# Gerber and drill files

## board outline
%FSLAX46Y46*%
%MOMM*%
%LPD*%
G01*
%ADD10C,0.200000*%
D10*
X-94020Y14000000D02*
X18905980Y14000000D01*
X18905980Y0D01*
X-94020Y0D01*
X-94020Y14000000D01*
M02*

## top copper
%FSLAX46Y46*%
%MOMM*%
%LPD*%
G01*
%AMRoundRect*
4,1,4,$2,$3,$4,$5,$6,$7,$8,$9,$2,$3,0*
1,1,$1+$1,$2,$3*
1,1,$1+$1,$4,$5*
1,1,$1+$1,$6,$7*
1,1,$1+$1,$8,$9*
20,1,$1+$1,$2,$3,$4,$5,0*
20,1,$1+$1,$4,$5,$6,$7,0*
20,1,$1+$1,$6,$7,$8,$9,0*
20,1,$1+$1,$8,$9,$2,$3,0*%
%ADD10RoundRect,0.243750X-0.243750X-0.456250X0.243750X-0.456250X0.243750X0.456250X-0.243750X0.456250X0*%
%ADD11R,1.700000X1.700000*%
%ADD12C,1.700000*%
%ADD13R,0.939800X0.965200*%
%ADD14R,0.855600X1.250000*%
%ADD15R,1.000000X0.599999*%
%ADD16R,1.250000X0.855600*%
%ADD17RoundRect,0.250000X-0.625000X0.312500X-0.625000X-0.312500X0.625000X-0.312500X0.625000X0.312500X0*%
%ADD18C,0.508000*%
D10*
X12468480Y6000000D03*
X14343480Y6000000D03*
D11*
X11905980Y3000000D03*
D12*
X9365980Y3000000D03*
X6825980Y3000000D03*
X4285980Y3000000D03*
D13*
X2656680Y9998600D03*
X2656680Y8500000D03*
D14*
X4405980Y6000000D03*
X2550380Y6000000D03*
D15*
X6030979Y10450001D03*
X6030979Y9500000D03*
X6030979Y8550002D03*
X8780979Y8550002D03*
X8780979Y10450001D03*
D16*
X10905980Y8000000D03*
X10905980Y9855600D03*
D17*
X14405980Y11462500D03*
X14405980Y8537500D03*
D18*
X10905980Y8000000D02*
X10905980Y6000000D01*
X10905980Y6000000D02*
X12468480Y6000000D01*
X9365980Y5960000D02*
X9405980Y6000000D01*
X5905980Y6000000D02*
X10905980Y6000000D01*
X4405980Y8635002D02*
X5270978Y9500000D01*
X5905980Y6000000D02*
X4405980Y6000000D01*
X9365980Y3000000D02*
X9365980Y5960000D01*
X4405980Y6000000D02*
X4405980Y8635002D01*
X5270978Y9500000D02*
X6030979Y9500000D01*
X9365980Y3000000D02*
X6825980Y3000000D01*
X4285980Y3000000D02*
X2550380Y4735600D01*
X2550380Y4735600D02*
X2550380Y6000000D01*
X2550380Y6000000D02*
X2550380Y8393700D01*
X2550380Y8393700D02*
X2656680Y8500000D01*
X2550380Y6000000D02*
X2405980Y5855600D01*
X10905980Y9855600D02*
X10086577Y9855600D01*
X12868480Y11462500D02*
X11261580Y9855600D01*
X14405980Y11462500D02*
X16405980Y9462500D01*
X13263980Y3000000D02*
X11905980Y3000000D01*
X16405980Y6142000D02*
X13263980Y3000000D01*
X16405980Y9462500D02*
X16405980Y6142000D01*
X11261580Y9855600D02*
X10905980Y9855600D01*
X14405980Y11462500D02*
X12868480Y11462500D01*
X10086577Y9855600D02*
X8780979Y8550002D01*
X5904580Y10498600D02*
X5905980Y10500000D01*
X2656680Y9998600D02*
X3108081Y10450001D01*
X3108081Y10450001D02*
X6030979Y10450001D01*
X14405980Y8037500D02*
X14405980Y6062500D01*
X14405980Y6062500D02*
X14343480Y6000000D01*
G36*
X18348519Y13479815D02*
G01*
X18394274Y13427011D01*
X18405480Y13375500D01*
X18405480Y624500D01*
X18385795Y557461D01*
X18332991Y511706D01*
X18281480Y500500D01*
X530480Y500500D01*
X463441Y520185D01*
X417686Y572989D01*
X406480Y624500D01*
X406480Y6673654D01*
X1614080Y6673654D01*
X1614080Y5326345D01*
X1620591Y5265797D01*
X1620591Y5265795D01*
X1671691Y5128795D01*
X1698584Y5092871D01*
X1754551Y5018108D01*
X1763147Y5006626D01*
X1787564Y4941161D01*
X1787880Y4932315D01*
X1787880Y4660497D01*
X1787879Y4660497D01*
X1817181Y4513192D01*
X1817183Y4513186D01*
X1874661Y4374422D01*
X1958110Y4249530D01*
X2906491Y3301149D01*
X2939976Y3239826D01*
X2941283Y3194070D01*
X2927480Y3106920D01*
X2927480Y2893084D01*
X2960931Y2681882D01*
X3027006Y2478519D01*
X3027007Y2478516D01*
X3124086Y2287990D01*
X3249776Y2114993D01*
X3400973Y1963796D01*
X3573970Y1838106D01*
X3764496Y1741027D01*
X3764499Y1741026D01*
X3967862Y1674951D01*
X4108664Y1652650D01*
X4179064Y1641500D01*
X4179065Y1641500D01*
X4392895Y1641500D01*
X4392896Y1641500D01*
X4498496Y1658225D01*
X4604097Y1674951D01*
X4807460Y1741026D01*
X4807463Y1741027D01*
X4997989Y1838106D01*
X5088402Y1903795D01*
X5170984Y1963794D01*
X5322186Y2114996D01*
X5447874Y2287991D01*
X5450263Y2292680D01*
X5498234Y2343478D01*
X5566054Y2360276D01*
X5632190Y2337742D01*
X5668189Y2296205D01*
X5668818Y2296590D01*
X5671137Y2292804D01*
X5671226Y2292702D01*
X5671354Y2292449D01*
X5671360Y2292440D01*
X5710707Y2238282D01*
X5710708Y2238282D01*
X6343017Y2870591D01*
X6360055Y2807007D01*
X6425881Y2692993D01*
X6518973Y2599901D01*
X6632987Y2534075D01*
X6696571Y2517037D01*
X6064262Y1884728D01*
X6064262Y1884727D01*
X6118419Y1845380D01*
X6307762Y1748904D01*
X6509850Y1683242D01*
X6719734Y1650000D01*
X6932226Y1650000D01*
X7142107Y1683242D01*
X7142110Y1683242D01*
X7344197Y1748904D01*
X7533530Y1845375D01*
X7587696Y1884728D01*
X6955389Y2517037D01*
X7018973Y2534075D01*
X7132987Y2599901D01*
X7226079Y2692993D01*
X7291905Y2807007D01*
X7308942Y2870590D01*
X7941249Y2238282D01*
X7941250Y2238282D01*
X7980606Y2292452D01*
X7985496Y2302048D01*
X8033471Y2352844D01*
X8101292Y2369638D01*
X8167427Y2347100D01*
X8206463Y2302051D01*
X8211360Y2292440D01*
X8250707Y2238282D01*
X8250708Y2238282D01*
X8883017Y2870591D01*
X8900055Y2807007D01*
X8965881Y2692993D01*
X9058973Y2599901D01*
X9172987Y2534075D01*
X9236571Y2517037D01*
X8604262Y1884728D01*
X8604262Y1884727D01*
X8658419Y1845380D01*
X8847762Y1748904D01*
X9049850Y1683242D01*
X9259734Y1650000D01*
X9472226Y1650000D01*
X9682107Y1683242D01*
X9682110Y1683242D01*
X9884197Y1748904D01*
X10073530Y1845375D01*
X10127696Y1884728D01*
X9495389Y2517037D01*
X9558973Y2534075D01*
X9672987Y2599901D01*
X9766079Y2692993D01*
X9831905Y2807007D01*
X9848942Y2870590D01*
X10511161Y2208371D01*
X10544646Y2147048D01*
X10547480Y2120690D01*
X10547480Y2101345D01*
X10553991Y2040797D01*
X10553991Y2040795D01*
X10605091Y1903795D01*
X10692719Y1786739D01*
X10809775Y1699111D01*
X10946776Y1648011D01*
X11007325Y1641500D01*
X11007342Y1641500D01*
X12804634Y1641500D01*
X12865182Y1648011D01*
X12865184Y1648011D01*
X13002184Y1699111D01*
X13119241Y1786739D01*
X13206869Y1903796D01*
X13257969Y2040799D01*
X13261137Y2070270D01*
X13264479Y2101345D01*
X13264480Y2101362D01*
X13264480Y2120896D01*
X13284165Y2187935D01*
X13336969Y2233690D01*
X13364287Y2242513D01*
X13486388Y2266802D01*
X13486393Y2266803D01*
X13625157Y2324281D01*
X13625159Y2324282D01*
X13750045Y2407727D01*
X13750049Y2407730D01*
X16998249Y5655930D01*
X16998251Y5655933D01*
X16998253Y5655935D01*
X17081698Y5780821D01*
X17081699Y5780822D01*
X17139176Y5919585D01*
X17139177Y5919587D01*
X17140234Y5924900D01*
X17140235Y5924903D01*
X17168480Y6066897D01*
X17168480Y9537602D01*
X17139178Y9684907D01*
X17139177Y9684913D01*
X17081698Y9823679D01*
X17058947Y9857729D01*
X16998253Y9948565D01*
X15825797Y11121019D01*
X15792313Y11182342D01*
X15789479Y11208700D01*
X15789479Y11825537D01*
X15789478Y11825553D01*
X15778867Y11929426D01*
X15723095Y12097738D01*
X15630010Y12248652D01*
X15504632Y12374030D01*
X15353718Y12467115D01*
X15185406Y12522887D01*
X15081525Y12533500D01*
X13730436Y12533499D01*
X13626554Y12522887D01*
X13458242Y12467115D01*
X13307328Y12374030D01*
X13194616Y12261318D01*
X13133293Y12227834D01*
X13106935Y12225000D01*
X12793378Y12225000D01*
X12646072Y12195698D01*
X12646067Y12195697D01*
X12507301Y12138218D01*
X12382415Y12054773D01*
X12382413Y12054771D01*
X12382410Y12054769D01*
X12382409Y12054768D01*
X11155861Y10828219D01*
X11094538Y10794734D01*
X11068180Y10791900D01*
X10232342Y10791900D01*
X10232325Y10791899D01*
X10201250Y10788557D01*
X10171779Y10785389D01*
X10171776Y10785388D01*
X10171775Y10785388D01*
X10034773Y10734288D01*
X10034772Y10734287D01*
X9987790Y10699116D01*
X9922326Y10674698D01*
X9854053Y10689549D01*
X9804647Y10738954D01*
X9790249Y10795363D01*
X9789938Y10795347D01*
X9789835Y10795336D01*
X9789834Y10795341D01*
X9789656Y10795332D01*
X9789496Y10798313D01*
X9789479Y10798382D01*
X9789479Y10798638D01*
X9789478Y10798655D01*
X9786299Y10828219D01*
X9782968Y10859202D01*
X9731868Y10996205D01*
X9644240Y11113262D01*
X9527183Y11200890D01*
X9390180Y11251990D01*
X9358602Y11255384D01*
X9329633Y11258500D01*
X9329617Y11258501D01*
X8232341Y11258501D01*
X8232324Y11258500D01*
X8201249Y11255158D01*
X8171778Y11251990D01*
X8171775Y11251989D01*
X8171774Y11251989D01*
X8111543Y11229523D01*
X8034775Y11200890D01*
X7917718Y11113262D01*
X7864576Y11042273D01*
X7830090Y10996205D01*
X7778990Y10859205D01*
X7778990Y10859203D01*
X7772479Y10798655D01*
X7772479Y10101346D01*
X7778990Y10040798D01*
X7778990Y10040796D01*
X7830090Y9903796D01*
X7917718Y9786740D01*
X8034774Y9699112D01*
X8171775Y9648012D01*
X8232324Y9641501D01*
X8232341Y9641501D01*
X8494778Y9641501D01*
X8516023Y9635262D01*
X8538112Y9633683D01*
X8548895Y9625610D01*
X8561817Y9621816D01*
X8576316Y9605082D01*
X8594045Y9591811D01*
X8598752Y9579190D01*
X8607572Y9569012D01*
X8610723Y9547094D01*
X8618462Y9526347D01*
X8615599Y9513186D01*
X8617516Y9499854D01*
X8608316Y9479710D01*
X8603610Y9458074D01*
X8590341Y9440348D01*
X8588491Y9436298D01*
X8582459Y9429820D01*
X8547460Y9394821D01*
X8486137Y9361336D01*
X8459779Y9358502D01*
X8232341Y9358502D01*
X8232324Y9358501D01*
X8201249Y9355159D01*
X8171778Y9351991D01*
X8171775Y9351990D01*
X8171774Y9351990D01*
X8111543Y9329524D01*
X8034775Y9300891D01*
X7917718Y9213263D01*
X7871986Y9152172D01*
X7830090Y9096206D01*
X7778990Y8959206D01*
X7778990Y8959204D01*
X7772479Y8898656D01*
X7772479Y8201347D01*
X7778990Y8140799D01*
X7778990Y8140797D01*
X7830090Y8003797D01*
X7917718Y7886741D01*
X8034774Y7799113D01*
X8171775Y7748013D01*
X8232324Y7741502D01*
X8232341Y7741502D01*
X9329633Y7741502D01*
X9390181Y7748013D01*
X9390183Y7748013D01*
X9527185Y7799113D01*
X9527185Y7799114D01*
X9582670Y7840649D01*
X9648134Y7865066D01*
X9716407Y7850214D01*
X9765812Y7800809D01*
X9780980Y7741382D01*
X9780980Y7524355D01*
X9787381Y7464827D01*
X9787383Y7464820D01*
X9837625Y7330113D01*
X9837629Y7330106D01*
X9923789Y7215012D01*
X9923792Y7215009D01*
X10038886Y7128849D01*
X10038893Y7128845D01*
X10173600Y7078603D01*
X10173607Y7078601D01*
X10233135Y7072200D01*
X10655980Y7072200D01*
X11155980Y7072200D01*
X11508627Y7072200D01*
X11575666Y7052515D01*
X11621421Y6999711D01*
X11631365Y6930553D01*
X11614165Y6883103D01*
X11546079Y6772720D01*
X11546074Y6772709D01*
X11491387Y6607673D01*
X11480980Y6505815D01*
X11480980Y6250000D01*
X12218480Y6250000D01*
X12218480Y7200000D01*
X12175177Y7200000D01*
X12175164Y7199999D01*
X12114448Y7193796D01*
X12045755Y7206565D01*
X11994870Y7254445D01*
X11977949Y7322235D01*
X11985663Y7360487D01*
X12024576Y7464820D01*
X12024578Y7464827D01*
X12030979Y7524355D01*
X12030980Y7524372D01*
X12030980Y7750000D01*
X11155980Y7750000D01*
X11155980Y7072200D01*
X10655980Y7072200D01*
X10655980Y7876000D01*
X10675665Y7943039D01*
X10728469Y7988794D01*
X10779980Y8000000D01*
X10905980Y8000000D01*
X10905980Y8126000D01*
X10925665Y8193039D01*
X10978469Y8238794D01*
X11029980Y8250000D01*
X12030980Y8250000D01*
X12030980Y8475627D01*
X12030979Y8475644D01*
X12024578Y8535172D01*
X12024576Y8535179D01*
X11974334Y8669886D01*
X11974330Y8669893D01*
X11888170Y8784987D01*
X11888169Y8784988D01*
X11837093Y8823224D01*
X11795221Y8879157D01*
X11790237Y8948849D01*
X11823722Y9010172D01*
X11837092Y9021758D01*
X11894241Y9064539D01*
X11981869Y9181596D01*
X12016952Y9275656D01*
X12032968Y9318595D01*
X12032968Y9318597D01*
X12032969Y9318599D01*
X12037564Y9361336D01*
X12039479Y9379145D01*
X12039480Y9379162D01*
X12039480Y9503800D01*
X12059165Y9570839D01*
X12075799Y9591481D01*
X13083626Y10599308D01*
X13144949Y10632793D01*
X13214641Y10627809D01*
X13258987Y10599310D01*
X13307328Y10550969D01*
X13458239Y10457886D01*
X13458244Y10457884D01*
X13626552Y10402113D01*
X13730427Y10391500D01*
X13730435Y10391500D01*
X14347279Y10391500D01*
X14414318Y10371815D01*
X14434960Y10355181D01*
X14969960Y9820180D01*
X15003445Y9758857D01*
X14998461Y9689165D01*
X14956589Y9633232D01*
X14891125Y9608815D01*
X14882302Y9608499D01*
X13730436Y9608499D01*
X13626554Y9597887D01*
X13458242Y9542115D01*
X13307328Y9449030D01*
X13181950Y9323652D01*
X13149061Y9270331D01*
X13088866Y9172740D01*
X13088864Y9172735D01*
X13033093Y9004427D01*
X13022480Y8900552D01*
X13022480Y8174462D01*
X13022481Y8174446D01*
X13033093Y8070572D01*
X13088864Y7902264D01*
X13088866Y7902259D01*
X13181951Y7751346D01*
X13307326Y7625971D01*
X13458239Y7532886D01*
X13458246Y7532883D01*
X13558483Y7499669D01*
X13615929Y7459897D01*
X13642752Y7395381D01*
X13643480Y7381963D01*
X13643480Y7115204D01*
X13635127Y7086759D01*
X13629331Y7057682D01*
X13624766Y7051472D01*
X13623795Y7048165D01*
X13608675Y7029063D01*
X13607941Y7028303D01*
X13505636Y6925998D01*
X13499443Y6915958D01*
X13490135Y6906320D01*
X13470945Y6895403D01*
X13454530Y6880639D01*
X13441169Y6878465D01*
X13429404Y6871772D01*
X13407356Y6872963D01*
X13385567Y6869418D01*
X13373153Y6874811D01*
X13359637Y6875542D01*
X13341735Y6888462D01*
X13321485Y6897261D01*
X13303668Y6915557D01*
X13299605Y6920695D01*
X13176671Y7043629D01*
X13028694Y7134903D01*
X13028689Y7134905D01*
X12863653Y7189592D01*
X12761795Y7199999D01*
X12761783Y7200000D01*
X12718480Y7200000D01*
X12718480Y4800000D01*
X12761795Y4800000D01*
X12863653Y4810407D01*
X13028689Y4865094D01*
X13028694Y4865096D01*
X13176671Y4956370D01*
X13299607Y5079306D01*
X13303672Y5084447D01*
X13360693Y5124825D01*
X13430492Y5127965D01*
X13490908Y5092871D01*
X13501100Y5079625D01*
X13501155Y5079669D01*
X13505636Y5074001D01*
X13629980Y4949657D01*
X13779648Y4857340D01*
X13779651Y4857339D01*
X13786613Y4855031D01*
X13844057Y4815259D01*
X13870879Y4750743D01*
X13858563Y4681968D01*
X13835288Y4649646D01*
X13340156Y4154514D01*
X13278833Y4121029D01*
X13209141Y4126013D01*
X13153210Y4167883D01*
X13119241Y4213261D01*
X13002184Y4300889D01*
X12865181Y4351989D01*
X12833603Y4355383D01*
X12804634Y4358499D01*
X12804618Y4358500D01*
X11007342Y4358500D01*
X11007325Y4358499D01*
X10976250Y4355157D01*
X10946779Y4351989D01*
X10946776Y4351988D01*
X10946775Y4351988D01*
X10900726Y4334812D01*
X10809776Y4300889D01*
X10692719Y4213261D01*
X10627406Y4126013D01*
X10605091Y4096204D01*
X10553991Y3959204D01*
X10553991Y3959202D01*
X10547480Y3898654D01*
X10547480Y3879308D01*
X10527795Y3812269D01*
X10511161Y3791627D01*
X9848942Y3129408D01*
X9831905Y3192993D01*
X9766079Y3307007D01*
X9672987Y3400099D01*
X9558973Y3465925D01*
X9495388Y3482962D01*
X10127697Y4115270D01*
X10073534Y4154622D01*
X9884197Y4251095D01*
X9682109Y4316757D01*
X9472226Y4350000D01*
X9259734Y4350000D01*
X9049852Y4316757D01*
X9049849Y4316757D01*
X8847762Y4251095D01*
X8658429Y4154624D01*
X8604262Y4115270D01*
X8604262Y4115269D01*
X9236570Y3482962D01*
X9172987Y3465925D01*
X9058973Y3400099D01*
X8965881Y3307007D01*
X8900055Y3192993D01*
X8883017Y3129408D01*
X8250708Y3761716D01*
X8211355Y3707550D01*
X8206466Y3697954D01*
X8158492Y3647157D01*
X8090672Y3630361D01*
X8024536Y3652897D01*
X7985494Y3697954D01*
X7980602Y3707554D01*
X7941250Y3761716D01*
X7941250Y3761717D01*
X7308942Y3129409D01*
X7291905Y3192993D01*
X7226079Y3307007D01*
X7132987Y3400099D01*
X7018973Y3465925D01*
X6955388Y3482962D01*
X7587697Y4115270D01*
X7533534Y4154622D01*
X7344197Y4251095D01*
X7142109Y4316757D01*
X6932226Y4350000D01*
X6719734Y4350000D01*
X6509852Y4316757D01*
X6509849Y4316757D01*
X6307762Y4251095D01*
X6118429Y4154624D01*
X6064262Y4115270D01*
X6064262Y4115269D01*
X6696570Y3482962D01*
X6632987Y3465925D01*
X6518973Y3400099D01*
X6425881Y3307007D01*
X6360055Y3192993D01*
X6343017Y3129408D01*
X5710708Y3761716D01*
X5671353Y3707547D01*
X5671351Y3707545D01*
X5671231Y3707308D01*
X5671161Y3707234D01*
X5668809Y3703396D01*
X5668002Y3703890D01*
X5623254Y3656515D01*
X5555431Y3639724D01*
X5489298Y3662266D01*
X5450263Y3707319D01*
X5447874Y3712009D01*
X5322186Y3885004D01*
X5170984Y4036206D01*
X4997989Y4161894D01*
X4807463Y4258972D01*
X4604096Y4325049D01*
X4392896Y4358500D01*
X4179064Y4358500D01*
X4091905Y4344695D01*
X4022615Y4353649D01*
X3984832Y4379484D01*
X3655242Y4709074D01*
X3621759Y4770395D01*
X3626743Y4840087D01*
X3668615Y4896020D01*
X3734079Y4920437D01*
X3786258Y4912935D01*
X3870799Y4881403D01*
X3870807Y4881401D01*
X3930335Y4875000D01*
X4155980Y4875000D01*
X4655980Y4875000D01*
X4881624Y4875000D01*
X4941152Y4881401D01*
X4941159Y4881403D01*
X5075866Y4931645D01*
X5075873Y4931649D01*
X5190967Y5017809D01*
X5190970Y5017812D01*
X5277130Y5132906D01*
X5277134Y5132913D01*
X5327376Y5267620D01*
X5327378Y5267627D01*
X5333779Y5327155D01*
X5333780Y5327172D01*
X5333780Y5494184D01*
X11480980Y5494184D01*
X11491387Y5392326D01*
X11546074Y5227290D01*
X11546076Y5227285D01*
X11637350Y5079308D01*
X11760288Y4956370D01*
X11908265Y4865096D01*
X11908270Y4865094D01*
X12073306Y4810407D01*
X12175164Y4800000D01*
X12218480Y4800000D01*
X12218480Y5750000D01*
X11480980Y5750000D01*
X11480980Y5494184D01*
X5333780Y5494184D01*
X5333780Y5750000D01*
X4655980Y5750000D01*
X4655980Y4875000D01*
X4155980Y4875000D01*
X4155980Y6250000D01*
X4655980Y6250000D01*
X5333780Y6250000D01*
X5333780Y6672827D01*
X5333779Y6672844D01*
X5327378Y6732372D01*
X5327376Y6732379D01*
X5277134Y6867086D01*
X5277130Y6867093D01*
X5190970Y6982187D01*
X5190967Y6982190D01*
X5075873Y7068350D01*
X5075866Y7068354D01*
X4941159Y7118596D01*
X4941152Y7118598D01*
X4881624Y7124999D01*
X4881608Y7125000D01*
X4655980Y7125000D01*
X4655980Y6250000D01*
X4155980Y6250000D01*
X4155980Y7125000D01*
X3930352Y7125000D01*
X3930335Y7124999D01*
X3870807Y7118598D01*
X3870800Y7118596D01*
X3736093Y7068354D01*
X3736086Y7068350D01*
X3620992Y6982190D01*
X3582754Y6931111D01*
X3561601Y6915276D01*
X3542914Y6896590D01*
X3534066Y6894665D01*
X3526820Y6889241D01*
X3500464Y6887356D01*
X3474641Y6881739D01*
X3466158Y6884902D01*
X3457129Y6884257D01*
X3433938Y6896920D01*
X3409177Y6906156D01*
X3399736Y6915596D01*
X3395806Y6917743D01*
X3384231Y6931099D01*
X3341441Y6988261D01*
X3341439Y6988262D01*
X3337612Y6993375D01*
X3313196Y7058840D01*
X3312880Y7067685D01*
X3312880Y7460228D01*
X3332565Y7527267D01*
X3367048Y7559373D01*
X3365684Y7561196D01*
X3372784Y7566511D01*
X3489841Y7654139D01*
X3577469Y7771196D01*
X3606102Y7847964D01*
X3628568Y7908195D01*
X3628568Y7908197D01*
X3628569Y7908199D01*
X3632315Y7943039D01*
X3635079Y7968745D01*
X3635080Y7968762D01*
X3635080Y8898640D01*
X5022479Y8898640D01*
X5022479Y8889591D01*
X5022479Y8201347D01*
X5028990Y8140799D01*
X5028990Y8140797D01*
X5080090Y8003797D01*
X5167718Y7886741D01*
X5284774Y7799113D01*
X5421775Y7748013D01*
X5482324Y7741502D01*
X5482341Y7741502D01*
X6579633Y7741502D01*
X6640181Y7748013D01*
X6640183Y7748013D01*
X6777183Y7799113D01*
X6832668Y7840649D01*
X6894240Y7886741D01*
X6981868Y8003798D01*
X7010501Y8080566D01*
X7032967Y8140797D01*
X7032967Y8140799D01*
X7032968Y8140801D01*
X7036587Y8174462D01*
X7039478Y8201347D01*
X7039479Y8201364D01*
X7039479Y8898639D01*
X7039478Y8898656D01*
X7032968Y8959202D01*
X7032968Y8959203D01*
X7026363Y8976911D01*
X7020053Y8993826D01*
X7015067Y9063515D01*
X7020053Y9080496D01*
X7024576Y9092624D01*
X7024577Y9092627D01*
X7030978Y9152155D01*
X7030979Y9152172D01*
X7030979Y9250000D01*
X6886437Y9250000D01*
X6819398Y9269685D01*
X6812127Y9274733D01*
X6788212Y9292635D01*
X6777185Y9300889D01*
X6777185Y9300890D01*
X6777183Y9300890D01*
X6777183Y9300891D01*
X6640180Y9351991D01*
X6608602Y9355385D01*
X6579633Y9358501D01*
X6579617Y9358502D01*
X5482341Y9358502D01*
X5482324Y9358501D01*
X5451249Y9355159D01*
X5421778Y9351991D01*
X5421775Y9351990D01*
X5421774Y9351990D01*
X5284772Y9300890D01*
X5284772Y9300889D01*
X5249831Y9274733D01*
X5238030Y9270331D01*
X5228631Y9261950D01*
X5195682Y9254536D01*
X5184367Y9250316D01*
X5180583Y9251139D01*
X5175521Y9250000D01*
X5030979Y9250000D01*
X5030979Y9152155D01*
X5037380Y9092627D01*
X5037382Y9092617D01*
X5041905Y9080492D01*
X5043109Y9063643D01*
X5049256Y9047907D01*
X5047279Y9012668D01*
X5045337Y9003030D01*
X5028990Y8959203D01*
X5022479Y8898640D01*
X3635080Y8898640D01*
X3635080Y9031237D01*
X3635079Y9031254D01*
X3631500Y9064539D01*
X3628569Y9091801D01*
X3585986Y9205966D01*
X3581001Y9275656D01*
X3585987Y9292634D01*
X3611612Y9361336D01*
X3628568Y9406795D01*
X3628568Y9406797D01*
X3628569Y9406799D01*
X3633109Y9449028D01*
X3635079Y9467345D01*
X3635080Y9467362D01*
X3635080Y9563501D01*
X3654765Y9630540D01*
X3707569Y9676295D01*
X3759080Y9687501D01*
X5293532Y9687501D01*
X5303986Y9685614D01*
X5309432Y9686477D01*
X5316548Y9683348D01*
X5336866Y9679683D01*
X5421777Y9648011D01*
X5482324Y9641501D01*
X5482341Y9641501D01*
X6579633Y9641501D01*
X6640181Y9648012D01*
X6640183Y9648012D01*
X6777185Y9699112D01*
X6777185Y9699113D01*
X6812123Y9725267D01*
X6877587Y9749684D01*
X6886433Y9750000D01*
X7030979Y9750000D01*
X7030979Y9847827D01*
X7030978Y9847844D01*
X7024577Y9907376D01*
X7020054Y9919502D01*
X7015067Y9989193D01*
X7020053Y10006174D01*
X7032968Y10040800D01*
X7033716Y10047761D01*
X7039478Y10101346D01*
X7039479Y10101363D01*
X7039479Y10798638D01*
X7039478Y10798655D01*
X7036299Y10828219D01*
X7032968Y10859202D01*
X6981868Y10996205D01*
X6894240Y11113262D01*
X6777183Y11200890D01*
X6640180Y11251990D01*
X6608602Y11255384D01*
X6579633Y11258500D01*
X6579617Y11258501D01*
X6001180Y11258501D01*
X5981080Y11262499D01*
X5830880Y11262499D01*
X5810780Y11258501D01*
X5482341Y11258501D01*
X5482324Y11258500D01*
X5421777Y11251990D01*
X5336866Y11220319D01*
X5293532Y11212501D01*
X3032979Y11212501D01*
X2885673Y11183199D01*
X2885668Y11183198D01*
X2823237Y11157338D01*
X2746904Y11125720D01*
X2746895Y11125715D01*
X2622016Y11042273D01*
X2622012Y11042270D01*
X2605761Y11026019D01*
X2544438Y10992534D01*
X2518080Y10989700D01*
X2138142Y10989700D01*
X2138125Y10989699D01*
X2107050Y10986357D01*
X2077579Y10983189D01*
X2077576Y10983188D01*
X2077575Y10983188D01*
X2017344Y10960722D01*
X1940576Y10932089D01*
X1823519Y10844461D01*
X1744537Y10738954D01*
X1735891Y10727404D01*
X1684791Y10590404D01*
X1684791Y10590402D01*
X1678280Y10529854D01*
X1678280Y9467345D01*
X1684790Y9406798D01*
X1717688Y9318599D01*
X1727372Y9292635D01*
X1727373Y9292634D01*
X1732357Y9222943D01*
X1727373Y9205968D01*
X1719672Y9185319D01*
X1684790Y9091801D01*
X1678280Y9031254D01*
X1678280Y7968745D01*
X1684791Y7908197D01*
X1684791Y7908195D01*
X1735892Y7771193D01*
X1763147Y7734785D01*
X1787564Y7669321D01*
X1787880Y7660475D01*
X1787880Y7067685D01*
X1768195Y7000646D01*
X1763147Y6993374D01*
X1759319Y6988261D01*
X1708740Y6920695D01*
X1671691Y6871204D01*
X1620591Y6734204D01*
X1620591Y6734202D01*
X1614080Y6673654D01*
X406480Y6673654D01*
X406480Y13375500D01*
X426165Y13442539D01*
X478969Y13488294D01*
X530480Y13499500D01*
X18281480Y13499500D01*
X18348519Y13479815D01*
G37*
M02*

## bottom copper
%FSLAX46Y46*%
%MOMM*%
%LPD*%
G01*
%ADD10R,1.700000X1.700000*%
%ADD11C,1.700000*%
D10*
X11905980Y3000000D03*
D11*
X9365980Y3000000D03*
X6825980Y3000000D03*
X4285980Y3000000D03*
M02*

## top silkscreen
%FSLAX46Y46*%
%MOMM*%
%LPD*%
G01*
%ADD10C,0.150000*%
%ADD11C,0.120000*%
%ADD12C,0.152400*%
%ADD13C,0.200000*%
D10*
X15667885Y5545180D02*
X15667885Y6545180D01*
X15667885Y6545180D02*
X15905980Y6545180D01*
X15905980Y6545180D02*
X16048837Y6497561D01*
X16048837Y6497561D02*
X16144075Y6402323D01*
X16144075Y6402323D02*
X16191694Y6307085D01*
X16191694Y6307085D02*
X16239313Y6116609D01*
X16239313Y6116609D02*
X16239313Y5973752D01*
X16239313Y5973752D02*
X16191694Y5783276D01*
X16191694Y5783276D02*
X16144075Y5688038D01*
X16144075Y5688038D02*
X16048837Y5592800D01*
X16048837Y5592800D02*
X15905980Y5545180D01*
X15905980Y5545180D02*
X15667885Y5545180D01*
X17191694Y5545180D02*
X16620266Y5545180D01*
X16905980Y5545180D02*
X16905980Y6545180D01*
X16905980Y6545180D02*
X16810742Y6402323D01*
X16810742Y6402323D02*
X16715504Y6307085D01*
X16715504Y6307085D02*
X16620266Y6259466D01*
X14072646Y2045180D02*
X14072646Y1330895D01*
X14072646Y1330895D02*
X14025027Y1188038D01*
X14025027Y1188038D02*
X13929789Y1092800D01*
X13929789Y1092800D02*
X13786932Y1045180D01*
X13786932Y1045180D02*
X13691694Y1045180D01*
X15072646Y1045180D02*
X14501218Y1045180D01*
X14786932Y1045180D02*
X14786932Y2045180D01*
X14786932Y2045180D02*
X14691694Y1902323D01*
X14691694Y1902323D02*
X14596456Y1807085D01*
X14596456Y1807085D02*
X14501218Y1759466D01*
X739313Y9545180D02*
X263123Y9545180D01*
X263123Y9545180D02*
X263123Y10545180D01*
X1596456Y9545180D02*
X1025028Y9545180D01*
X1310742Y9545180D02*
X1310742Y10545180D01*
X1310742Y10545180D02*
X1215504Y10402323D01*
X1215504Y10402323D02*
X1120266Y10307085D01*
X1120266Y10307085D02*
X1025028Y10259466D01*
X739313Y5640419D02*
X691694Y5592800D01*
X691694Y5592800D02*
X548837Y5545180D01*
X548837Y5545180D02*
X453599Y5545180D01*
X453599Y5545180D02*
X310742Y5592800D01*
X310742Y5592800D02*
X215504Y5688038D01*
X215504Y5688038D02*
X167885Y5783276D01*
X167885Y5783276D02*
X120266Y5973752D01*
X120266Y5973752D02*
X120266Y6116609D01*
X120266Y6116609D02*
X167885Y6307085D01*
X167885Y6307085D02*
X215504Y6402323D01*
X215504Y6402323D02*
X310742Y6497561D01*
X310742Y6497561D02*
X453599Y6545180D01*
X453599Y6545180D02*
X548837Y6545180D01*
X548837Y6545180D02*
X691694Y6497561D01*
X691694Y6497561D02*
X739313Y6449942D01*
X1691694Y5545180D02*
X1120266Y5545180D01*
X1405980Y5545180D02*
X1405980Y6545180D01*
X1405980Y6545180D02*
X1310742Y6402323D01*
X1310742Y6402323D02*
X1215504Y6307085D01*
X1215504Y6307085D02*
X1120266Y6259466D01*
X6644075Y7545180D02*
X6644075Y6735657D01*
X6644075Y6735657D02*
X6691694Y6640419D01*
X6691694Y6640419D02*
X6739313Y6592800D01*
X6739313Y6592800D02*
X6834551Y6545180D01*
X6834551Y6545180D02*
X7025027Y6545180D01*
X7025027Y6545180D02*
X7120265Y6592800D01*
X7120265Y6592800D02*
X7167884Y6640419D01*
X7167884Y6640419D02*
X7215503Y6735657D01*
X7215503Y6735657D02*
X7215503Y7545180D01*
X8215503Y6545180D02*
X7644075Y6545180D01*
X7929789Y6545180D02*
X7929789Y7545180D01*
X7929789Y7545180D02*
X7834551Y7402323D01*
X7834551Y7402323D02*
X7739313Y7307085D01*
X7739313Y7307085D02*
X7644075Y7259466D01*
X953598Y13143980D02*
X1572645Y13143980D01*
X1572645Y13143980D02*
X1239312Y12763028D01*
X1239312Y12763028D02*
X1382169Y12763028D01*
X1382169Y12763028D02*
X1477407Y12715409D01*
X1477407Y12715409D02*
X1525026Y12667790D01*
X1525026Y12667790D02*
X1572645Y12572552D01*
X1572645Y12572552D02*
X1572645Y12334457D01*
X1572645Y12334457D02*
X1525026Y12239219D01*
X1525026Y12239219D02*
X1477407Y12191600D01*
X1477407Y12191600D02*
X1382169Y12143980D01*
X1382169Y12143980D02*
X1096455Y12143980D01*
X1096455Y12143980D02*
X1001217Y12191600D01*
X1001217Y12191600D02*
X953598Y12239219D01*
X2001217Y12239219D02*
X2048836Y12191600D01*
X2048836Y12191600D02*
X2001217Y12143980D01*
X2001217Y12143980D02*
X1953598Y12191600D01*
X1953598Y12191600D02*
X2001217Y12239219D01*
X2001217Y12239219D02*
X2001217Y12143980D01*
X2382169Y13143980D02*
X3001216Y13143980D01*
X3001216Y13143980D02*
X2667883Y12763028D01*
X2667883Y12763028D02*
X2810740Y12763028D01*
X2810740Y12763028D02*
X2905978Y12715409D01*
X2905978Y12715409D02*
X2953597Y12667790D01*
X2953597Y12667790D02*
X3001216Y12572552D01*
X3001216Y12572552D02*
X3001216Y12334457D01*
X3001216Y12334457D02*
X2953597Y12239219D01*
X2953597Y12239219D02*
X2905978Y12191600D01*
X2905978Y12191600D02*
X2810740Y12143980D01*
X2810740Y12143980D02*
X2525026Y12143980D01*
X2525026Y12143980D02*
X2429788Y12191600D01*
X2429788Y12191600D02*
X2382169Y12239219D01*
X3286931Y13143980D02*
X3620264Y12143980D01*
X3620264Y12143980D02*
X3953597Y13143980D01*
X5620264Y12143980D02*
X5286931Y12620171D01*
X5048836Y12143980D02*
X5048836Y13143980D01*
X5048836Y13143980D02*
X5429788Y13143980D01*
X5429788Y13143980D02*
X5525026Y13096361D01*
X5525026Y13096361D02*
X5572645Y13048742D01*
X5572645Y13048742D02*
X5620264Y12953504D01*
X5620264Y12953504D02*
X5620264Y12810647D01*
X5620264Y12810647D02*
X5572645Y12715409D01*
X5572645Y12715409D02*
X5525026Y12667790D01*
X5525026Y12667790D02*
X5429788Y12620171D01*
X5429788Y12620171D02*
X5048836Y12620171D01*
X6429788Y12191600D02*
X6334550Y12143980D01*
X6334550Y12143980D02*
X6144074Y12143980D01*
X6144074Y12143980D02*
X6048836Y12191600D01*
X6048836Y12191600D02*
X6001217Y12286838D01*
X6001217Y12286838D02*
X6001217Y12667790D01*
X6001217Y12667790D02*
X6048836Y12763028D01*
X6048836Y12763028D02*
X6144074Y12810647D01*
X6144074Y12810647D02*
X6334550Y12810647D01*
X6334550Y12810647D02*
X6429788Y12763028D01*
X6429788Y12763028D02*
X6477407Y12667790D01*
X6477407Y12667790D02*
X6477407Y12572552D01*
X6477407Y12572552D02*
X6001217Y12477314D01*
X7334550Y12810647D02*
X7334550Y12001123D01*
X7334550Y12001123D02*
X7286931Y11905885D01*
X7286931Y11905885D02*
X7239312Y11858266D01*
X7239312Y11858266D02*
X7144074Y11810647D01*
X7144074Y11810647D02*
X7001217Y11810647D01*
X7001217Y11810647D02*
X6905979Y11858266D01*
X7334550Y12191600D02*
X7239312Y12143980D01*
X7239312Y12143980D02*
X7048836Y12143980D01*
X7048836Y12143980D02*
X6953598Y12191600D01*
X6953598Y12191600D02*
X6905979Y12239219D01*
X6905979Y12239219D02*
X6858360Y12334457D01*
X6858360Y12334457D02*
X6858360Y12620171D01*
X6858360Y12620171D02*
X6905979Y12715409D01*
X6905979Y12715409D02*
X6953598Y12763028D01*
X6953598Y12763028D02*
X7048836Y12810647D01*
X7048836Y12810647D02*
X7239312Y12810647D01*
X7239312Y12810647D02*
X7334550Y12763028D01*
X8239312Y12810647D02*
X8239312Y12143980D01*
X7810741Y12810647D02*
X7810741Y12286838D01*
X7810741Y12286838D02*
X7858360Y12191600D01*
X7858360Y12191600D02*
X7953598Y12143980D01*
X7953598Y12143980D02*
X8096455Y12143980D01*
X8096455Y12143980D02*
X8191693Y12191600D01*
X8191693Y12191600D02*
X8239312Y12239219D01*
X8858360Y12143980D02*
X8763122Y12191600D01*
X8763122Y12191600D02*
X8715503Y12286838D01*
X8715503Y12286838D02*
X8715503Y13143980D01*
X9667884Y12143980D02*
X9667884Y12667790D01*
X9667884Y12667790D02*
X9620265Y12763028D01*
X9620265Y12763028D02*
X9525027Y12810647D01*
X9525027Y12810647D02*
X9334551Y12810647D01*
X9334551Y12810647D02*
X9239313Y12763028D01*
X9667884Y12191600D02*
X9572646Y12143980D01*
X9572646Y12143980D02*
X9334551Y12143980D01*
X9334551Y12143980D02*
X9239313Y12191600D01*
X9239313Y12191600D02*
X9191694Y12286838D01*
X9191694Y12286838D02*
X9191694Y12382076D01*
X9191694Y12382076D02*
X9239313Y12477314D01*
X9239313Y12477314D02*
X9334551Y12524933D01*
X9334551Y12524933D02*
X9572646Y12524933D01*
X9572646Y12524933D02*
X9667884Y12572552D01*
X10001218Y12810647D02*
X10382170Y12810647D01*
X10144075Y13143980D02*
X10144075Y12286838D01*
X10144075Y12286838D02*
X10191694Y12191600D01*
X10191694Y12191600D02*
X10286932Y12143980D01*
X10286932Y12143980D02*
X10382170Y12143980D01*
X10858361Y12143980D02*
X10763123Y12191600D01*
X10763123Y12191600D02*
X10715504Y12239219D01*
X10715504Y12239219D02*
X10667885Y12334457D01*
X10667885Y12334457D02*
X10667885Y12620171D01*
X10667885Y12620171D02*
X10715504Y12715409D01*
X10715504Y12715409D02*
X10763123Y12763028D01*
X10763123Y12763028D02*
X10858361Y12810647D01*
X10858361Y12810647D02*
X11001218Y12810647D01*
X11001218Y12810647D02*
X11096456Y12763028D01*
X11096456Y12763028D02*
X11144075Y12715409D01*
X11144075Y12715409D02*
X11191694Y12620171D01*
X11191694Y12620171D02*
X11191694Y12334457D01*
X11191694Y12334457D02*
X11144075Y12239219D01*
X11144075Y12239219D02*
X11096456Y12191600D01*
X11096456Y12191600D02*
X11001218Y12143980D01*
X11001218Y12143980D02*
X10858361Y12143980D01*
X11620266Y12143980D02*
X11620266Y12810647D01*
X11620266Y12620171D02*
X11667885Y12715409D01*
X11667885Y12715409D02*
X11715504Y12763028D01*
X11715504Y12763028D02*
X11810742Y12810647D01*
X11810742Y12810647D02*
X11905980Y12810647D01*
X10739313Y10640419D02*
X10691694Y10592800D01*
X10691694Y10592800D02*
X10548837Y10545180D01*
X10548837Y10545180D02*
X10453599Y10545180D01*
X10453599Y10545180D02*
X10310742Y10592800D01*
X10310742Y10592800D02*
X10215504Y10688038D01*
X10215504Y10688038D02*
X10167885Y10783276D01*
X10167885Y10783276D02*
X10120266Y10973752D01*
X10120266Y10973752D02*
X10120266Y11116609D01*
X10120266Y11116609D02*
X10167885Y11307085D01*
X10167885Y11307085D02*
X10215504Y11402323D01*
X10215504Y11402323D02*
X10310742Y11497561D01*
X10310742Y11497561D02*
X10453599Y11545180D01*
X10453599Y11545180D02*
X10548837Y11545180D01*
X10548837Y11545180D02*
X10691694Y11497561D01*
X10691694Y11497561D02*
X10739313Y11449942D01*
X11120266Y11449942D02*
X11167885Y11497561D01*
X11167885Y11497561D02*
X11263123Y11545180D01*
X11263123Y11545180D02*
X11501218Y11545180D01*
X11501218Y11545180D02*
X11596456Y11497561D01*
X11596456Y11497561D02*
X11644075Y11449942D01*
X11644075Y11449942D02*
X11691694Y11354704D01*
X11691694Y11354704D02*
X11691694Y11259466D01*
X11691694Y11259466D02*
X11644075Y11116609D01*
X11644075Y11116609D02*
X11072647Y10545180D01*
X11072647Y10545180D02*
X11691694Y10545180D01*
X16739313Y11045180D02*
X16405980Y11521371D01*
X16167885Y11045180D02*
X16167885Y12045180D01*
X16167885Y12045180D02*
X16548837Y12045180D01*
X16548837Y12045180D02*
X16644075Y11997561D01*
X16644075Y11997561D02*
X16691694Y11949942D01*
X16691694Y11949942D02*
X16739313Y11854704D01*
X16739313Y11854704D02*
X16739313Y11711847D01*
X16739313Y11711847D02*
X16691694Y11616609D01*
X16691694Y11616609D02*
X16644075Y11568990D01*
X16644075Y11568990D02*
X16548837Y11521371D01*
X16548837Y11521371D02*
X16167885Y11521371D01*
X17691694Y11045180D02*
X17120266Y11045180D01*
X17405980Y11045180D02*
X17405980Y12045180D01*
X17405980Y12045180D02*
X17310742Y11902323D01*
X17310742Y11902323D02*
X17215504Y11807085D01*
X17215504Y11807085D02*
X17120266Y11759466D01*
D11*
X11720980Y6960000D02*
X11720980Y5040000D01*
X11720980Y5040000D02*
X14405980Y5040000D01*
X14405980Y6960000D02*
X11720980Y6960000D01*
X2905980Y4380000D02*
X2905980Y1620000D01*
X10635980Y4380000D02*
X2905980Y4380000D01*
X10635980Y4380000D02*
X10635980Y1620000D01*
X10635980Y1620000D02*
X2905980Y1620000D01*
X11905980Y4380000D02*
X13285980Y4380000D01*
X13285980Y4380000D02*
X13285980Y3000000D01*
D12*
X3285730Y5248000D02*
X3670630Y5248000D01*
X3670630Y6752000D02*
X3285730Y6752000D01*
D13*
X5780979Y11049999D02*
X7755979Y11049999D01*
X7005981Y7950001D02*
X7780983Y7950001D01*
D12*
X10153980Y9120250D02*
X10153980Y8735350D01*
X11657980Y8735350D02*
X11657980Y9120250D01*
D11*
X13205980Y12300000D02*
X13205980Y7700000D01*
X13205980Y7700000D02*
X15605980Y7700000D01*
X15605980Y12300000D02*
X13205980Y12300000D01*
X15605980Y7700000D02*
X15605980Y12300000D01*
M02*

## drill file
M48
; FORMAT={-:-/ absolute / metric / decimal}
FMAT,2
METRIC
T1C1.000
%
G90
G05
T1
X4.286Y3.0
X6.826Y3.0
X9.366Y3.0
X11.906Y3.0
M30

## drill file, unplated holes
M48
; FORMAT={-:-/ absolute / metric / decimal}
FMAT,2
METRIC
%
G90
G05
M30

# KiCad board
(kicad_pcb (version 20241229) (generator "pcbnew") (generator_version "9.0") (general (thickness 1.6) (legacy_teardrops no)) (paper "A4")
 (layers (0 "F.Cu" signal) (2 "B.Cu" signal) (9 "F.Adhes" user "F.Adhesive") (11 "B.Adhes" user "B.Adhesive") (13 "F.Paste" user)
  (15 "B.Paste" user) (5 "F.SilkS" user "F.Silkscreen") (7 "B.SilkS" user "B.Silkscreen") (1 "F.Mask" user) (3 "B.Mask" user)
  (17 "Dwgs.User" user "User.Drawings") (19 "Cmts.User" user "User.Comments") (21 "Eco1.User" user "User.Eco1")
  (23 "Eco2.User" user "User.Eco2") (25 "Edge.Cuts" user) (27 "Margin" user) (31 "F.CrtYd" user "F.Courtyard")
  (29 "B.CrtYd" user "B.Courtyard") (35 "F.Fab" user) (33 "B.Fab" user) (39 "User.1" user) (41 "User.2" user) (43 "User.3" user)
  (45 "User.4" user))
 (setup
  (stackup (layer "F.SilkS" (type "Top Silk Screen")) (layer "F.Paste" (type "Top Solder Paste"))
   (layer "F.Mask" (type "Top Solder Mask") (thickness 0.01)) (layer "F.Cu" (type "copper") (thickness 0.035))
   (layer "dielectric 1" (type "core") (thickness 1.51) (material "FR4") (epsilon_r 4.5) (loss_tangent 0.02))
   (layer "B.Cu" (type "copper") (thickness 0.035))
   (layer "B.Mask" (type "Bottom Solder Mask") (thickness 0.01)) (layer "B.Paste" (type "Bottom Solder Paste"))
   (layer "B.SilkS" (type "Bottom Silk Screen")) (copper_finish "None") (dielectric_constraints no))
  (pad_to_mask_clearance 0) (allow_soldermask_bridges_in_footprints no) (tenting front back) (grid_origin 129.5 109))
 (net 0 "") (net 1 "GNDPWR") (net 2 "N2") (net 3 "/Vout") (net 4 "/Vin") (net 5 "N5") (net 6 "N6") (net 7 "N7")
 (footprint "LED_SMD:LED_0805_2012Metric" (layer "F.Cu") (at 13.40598 -6)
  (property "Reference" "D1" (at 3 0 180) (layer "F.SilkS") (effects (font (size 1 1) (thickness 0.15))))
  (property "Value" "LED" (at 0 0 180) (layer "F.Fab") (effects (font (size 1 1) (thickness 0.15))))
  (fp_line (start -1.685 -0.96) (end -1.685 0.96) (stroke (width 0.12) (type solid)) (layer "F.SilkS"))
  (fp_line (start -1.685 0.96) (end 1 0.96) (stroke (width 0.12) (type solid)) (layer "F.SilkS"))
  (fp_line (start 1 -0.96) (end -1.685 -0.96) (stroke (width 0.12) (type solid)) (layer "F.SilkS"))
  (pad "1" smd roundrect (at -0.9375 0) (size 0.975 1.4) (layers "F.Cu" "F.Mask" "F.Paste") (roundrect_rratio 0.25) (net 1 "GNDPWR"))
  (pad "2" smd roundrect (at 0.9375 0) (size 0.975 1.4) (layers "F.Cu" "F.Mask" "F.Paste") (roundrect_rratio 0.25) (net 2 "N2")))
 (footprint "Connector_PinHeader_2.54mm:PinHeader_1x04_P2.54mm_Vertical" (layer "F.Cu") (at 11.90598 -3 -90)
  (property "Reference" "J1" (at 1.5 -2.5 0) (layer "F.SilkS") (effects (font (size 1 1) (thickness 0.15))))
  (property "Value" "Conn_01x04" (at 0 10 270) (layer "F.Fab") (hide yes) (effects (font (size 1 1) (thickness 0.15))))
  (fp_line (start -1.38 9) (end 1.38 9) (stroke (width 0.12) (type solid)) (layer "F.SilkS"))
  (fp_line (start -1.38 1.27) (end -1.38 9) (stroke (width 0.12) (type solid)) (layer "F.SilkS"))
  (fp_line (start -1.38 1.27) (end 1.38 1.27) (stroke (width 0.12) (type solid)) (layer "F.SilkS"))
  (fp_line (start 1.38 1.27) (end 1.38 9) (stroke (width 0.12) (type solid)) (layer "F.SilkS"))
  (fp_line (start -1.38 0) (end -1.38 -1.38) (stroke (width 0.12) (type solid)) (layer "F.SilkS"))
  (fp_line (start -1.38 -1.38) (end 0 -1.38) (stroke (width 0.12) (type solid)) (layer "F.SilkS"))
  (pad "1" thru_hole rect (at 0 0 270) (size 1.7 1.7) (drill 1) (layers "*.Cu" "*.Mask") (remove_unused_layers no) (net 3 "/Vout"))
  (pad "2" thru_hole circle (at 0 2.54 270) (size 1.7 1.7) (drill 1) (layers "*.Cu" "*.Mask") (remove_unused_layers no) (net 1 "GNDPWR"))
  (pad "3" thru_hole circle (at 0 5.08 270) (size 1.7 1.7) (drill 1) (layers "*.Cu" "*.Mask") (remove_unused_layers no) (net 1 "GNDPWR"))
  (pad "4" thru_hole circle (at 0 7.62 270) (size 1.7 1.7) (drill 1) (layers "*.Cu" "*.Mask") (remove_unused_layers no) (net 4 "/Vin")))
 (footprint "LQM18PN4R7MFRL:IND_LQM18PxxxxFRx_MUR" (layer "F.Cu") (at 2.65668 -9.2493 -90)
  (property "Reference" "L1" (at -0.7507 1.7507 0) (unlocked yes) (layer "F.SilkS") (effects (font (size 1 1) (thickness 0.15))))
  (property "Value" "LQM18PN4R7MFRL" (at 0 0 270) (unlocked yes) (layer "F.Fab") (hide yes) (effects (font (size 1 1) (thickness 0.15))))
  (pad "1" smd rect (at -0.7493 0 270) (size 0.9652 0.9398) (layers "F.Cu" "F.Mask" "F.Paste") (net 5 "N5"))
  (pad "2" smd rect (at 0.7493 0 270) (size 0.9652 0.9398) (layers "F.Cu" "F.Mask" "F.Paste") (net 4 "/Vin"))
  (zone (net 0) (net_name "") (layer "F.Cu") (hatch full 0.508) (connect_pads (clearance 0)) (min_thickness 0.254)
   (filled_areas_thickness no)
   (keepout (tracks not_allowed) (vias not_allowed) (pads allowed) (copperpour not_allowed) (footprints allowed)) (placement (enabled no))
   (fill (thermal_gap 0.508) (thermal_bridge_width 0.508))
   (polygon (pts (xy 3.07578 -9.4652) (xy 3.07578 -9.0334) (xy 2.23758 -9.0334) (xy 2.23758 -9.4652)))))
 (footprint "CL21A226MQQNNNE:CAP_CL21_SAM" (layer "F.Cu") (at 3.47818 -6 180)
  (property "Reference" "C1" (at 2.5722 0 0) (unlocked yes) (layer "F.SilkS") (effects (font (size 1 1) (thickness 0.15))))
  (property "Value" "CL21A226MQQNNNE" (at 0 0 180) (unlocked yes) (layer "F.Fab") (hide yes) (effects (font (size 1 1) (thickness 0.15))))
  (fp_line (start 0.19245 -0.752) (end -0.19245 -0.752) (stroke (width 0.1524) (type solid)) (layer "F.SilkS"))
  (fp_line (start -0.19245 0.752) (end 0.19245 0.752) (stroke (width 0.1524) (type solid)) (layer "F.SilkS"))
  (pad "1" smd rect (at -0.9278 0 180) (size 0.8556 1.25) (layers "F.Cu" "F.Mask" "F.Paste") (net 1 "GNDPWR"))
  (pad "2" smd rect (at 0.9278 0 180) (size 0.8556 1.25) (layers "F.Cu" "F.Mask" "F.Paste") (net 4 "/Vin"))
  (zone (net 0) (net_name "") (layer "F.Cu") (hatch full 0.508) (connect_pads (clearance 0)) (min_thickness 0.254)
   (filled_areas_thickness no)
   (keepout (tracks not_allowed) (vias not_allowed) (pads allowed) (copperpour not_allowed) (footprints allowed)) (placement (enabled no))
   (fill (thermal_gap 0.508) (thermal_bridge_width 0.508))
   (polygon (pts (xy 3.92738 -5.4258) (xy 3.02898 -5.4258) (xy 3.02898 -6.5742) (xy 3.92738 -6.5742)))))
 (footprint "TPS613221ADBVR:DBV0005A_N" (layer "F.Cu") (at 7.40598 -9.5)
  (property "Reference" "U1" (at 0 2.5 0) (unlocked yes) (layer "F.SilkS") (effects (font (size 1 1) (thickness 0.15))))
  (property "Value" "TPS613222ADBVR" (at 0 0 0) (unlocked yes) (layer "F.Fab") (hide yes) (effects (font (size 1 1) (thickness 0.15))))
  (fp_line (start -1.625001 -1.549999) (end 0.349999 -1.549999) (stroke (width 0.2) (type solid)) (layer "F.SilkS"))
  (fp_line (start -0.399999 1.549999) (end 0.375003 1.549999) (stroke (width 0.2) (type solid)) (layer "F.SilkS"))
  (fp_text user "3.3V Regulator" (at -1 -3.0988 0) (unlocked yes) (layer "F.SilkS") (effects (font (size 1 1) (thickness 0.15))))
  (pad "1" smd rect (at -1.375001 -0.950001 90) (size 0.599999 1) (layers "F.Cu" "F.Mask" "F.Paste") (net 5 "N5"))
  (pad "2" smd rect (at -1.375001 0 90) (size 0.599999 1) (layers "F.Cu" "F.Mask" "F.Paste") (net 1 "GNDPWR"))
  (pad "3" smd rect (at -1.375001 0.949998 90) (size 0.599999 1) (layers "F.Cu" "F.Mask" "F.Paste") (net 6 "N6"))
  (pad "4" smd rect (at 1.374999 0.949998 90) (size 0.599999 1) (layers "F.Cu" "F.Mask" "F.Paste") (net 3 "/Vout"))
  (pad "5" smd rect (at 1.374999 -0.950001 90) (size 0.599999 1) (layers "F.Cu" "F.Mask" "F.Paste") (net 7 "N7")))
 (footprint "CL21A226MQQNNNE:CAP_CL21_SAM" (layer "F.Cu") (at 10.90598 -8.9278 90)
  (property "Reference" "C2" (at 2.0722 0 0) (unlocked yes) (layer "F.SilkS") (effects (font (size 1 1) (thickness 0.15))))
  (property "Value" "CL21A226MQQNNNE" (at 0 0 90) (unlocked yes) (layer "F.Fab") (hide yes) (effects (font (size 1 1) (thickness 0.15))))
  (fp_line (start 0.19245 -0.752) (end -0.19245 -0.752) (stroke (width 0.1524) (type solid)) (layer "F.SilkS"))
  (fp_line (start -0.19245 0.752) (end 0.19245 0.752) (stroke (width 0.1524) (type solid)) (layer "F.SilkS"))
  (pad "1" smd rect (at -0.9278 0 90) (size 0.8556 1.25) (layers "F.Cu" "F.Mask" "F.Paste") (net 1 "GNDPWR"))
  (pad "2" smd rect (at 0.9278 0 90) (size 0.8556 1.25) (layers "F.Cu" "F.Mask" "F.Paste") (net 3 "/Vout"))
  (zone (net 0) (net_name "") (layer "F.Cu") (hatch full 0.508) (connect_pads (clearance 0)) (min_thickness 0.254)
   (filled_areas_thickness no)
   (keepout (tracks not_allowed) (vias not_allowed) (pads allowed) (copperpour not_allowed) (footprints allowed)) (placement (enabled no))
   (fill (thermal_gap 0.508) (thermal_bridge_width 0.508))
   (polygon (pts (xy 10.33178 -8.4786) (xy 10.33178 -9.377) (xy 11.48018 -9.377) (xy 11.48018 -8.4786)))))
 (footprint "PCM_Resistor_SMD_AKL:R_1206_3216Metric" (layer "F.Cu") (at 14.40598 -10 -90)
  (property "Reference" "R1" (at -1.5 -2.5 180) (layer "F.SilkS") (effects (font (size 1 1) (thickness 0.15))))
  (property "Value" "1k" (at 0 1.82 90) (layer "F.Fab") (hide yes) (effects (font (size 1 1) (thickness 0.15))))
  (fp_line (start -2.3 1.2) (end 2.3 1.2) (stroke (width 0.12) (type solid)) (layer "F.SilkS"))
  (fp_line (start 2.3 1.2) (end 2.3 -1.2) (stroke (width 0.12) (type solid)) (layer "F.SilkS"))
  (fp_line (start -2.3 -1.2) (end -2.3 1.2) (stroke (width 0.12) (type solid)) (layer "F.SilkS"))
  (fp_line (start 2.3 -1.2) (end -2.3 -1.2) (stroke (width 0.12) (type solid)) (layer "F.SilkS"))
  (pad "1" smd roundrect (at -1.4625 0 270) (size 1.125 1.75) (layers "F.Cu" "F.Mask" "F.Paste") (roundrect_rratio 0.222222) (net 3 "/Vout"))
  (pad "2" smd roundrect (at 1.4625 0 270) (size 1.125 1.75) (layers "F.Cu" "F.Mask" "F.Paste") (roundrect_rratio 0.222222) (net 2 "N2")))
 (gr_rect (start -0.09402 -14) (end 18.90598 0) (stroke (width 0.2) (type solid)) (fill no) (layer "Edge.Cuts"))
 (segment (start 10.90598 -8) (end 10.90598 -6) (width 0.508) (layer "F.Cu") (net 1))
 (segment (start 10.90598 -6) (end 12.46848 -6) (width 0.508) (layer "F.Cu") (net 1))
 (segment (start 9.36598 -5.96) (end 9.40598 -6) (width 0.508) (layer "F.Cu") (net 1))
 (segment (start 5.90598 -6) (end 10.90598 -6) (width 0.508) (layer "F.Cu") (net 1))
 (segment (start 4.40598 -8.635002) (end 5.270978 -9.5) (width 0.508) (layer "F.Cu") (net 1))
 (segment (start 5.90598 -6) (end 4.40598 -6) (width 0.508) (layer "F.Cu") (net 1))
 (segment (start 9.36598 -3) (end 9.36598 -5.96) (width 0.508) (layer "F.Cu") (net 1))
 (segment (start 4.40598 -6) (end 4.40598 -8.635002) (width 0.508) (layer "F.Cu") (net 1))
 (segment (start 5.270978 -9.5) (end 6.030979 -9.5) (width 0.508) (layer "F.Cu") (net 1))
 (segment (start 9.36598 -3) (end 6.82598 -3) (width 0.508) (layer "F.Cu") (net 1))
 (segment (start 4.28598 -3) (end 2.55038 -4.7356) (width 0.508) (layer "F.Cu") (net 4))
 (segment (start 2.55038 -4.7356) (end 2.55038 -6) (width 0.508) (layer "F.Cu") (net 4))
 (segment (start 2.55038 -6) (end 2.55038 -8.3937) (width 0.508) (layer "F.Cu") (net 4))
 (segment (start 2.55038 -8.3937) (end 2.65668 -8.5) (width 0.508) (layer "F.Cu") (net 4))
 (segment (start 2.55038 -6) (end 2.40598 -5.8556) (width 0.508) (layer "F.Cu") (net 4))
 (segment (start 10.90598 -9.8556) (end 10.086577 -9.8556) (width 0.508) (layer "F.Cu") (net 3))
 (segment (start 12.86848 -11.4625) (end 11.26158 -9.8556) (width 0.508) (layer "F.Cu") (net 3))
 (segment (start 14.40598 -11.4625) (end 16.40598 -9.4625) (width 0.508) (layer "F.Cu") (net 3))
 (segment (start 13.26398 -3) (end 11.90598 -3) (width 0.508) (layer "F.Cu") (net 3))
 (segment (start 16.40598 -6.142) (end 13.26398 -3) (width 0.508) (layer "F.Cu") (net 3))
 (segment (start 16.40598 -9.4625) (end 16.40598 -6.142) (width 0.508) (layer "F.Cu") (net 3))
 (segment (start 11.26158 -9.8556) (end 10.90598 -9.8556) (width 0.508) (layer "F.Cu") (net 3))
 (segment (start 14.40598 -11.4625) (end 12.86848 -11.4625) (width 0.508) (layer "F.Cu") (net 3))
 (segment (start 10.086577 -9.8556) (end 8.780979 -8.550002) (width 0.508) (layer "F.Cu") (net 3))
 (segment (start 5.90458 -10.4986) (end 5.90598 -10.5) (width 0.508) (layer "F.Cu") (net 5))
 (segment (start 2.65668 -9.9986) (end 3.108081 -10.450001) (width 0.508) (layer "F.Cu") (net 5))
 (segment (start 3.108081 -10.450001) (end 6.030979 -10.450001) (width 0.508) (layer "F.Cu") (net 5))
 (segment (start 14.40598 -8.0375) (end 14.40598 -6.0625) (width 0.508) (layer "F.Cu") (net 2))
 (segment (start 14.40598 -6.0625) (end 14.34348 -6) (width 0.508) (layer "F.Cu") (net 2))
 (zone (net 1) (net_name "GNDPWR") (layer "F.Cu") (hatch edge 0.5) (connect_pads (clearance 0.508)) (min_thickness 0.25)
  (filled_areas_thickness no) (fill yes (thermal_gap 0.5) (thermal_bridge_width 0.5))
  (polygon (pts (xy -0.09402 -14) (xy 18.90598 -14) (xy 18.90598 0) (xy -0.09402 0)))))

